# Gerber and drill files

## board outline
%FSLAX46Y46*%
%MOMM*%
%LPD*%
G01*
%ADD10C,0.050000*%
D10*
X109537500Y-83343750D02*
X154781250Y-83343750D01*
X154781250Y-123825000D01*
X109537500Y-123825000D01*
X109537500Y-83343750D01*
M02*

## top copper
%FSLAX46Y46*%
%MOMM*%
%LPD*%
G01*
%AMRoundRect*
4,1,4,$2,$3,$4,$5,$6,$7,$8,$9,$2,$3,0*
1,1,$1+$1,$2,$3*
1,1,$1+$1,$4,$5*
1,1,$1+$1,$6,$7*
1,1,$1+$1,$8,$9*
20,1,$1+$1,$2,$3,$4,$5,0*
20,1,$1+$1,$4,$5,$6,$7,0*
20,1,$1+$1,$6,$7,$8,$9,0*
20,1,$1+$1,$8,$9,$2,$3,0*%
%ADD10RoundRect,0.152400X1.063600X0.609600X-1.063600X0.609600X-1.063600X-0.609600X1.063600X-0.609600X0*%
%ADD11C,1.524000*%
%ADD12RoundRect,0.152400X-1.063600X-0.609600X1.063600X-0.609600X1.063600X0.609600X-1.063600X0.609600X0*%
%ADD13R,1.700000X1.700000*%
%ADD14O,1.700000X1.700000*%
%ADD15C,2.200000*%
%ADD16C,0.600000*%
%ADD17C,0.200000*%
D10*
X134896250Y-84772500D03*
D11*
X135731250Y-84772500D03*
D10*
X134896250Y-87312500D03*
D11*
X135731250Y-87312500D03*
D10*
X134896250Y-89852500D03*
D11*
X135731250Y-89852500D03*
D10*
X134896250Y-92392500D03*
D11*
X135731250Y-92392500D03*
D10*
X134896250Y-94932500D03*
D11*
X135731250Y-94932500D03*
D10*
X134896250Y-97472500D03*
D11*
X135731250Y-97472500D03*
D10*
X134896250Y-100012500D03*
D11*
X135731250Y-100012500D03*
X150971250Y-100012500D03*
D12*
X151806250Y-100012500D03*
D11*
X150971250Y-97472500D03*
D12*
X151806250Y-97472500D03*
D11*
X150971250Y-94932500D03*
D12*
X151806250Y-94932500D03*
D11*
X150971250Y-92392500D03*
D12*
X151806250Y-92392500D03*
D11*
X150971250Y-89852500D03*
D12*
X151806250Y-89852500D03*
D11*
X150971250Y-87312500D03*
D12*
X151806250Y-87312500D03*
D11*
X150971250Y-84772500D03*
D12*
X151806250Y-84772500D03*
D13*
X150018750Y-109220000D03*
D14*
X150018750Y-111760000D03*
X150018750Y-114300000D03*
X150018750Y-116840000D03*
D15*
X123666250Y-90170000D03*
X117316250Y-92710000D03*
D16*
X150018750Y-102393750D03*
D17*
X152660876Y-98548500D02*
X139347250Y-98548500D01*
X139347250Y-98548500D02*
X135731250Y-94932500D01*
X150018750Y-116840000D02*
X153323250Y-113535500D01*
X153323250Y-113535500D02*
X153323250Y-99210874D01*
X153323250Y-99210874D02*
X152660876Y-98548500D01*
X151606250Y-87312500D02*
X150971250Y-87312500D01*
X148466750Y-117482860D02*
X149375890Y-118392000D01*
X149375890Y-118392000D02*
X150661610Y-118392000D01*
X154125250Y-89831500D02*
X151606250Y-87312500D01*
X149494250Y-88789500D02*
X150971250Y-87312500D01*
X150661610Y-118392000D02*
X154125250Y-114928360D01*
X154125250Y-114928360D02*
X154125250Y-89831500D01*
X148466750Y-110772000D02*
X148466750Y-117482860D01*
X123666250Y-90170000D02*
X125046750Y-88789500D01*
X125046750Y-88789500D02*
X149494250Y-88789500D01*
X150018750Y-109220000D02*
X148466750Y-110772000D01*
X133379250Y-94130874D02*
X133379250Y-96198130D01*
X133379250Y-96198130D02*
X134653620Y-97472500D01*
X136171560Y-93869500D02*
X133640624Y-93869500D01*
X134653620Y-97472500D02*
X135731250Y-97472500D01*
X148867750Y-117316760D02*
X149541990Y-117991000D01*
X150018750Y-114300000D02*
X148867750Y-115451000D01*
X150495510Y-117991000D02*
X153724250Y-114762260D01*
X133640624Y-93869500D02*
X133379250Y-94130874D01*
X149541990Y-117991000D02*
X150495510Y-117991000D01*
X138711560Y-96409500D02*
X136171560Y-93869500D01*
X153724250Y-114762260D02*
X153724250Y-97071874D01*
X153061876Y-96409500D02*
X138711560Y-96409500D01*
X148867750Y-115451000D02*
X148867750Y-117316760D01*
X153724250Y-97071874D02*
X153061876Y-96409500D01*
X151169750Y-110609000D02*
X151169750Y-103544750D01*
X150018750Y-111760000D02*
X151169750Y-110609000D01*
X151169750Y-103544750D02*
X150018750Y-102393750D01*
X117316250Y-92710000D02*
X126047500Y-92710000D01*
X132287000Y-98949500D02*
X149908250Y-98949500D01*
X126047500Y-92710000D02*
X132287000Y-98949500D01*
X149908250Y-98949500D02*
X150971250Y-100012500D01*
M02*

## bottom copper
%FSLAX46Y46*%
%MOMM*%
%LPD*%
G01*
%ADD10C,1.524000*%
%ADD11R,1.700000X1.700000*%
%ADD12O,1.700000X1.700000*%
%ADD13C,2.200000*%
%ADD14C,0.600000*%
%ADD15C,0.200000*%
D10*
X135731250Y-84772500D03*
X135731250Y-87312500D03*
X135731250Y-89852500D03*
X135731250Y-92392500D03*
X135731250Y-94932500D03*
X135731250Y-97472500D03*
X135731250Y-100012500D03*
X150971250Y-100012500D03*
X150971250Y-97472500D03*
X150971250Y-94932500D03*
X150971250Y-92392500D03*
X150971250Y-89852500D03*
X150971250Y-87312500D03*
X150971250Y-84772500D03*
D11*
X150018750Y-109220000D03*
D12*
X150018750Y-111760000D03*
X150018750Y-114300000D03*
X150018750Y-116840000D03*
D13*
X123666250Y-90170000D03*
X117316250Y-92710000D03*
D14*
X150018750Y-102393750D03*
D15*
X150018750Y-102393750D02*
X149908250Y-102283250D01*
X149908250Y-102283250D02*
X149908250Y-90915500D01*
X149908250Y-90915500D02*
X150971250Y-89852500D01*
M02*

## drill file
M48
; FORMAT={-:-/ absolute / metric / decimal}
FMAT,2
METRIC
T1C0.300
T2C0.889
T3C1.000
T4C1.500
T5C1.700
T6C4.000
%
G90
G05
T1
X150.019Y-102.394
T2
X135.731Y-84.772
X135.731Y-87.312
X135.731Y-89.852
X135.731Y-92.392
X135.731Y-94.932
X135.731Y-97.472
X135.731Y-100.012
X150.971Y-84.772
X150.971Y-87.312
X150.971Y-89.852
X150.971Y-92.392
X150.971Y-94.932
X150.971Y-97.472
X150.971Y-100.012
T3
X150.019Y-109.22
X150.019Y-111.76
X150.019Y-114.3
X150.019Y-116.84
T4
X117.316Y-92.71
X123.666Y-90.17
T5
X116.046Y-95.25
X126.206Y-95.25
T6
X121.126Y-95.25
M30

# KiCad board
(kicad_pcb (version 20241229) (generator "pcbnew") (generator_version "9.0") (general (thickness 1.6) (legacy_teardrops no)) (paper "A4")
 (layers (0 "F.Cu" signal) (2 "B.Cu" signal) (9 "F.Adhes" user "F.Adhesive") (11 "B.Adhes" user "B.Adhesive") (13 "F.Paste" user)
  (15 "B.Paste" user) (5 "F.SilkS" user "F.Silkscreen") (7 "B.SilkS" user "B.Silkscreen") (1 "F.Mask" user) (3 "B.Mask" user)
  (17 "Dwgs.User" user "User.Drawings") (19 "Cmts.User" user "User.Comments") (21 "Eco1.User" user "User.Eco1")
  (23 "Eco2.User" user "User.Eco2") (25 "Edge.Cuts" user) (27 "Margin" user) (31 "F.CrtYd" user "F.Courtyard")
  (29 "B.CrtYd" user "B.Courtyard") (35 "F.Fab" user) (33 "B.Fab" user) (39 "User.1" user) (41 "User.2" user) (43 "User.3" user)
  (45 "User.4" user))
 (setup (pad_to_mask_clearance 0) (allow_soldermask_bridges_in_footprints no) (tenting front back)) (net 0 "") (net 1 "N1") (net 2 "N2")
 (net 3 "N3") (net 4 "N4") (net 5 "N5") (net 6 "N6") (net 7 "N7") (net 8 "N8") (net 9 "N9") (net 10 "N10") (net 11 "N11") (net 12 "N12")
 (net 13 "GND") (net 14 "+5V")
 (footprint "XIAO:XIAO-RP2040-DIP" (layer "F.Cu") (at 143.35125 92.3925)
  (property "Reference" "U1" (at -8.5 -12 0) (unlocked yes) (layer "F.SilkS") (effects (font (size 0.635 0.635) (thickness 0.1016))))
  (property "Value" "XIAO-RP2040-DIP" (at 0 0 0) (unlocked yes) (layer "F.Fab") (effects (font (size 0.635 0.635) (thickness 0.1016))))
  (pad "1" smd roundrect (at -8.455 -7.62 180) (size 2.432 1.524) (layers "F.Cu" "F.Mask") (roundrect_rratio 0.1) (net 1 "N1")
   (thermal_bridge_angle 45))
  (pad "1" thru_hole circle (at -7.62 -7.62 180) (size 1.524 1.524) (drill 0.889) (layers "*.Cu" "*.Mask") (remove_unused_layers no)
   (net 1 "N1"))
  (pad "2" smd roundrect (at -8.455 -5.08 180) (size 2.432 1.524) (layers "F.Cu" "F.Mask") (roundrect_rratio 0.1) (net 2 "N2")
   (thermal_bridge_angle 45))
  (pad "2" thru_hole circle (at -7.62 -5.08 180) (size 1.524 1.524) (drill 0.889) (layers "*.Cu" "*.Mask") (remove_unused_layers no)
   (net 2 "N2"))
  (pad "3" smd roundrect (at -8.455 -2.54 180) (size 2.432 1.524) (layers "F.Cu" "F.Mask") (roundrect_rratio 0.1) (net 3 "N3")
   (thermal_bridge_angle 45))
  (pad "3" thru_hole circle (at -7.62 -2.54 180) (size 1.524 1.524) (drill 0.889) (layers "*.Cu" "*.Mask") (remove_unused_layers no)
   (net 3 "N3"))
  (pad "4" smd roundrect (at -8.455 0 180) (size 2.432 1.524) (layers "F.Cu" "F.Mask") (roundrect_rratio 0.1) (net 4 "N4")
   (thermal_bridge_angle 45))
  (pad "4" thru_hole circle (at -7.62 0 180) (size 1.524 1.524) (drill 0.889) (layers "*.Cu" "*.Mask") (remove_unused_layers no)
   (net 4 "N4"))
  (pad "5" smd roundrect (at -8.455 2.54 180) (size 2.432 1.524) (layers "F.Cu" "F.Mask") (roundrect_rratio 0.1) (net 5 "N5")
   (thermal_bridge_angle 45))
  (pad "5" thru_hole circle (at -7.62 2.54 180) (size 1.524 1.524) (drill 0.889) (layers "*.Cu" "*.Mask") (remove_unused_layers no)
   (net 5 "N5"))
  (pad "6" smd roundrect (at -8.455 5.08 180) (size 2.432 1.524) (layers "F.Cu" "F.Mask") (roundrect_rratio 0.1) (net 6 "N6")
   (thermal_bridge_angle 45))
  (pad "6" thru_hole circle (at -7.62 5.08 180) (size 1.524 1.524) (drill 0.889) (layers "*.Cu" "*.Mask") (remove_unused_layers no)
   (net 6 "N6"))
  (pad "7" smd roundrect (at -8.455 7.62 180) (size 2.432 1.524) (layers "F.Cu" "F.Mask") (roundrect_rratio 0.1) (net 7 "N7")
   (thermal_bridge_angle 45))
  (pad "7" thru_hole circle (at -7.62 7.62 180) (size 1.524 1.524) (drill 0.889) (layers "*.Cu" "*.Mask") (remove_unused_layers no)
   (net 7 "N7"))
  (pad "8" thru_hole circle (at 7.62 7.62) (size 1.524 1.524) (drill 0.889) (layers "*.Cu" "*.Mask") (remove_unused_layers no) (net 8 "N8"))
  (pad "8" smd roundrect (at 8.455 7.62) (size 2.432 1.524) (layers "F.Cu" "F.Mask") (roundrect_rratio 0.1) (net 8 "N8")
   (thermal_bridge_angle 45))
  (pad "9" thru_hole circle (at 7.62 5.08) (size 1.524 1.524) (drill 0.889) (layers "*.Cu" "*.Mask") (remove_unused_layers no) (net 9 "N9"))
  (pad "9" smd roundrect (at 8.455 5.08) (size 2.432 1.524) (layers "F.Cu" "F.Mask") (roundrect_rratio 0.1) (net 9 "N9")
   (thermal_bridge_angle 45))
  (pad "10" thru_hole circle (at 7.62 2.54) (size 1.524 1.524) (drill 0.889) (layers "*.Cu" "*.Mask") (remove_unused_layers no)
   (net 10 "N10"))
  (pad "10" smd roundrect (at 8.455 2.54) (size 2.432 1.524) (layers "F.Cu" "F.Mask") (roundrect_rratio 0.1) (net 10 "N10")
   (thermal_bridge_angle 45))
  (pad "11" thru_hole circle (at 7.62 0) (size 1.524 1.524) (drill 0.889) (layers "*.Cu" "*.Mask") (remove_unused_layers no) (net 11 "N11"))
  (pad "11" smd roundrect (at 8.455 0) (size 2.432 1.524) (layers "F.Cu" "F.Mask") (roundrect_rratio 0.1) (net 11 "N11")
   (thermal_bridge_angle 45))
  (pad "12" thru_hole circle (at 7.62 -2.54) (size 1.524 1.524) (drill 0.889) (layers "*.Cu" "*.Mask") (remove_unused_layers no)
   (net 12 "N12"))
  (pad "12" smd roundrect (at 8.455 -2.54) (size 2.432 1.524) (layers "F.Cu" "F.Mask") (roundrect_rratio 0.1) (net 12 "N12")
   (thermal_bridge_angle 45))
  (pad "13" thru_hole circle (at 7.62 -5.08) (size 1.524 1.524) (drill 0.889) (layers "*.Cu" "*.Mask") (remove_unused_layers no)
   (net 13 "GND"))
  (pad "13" smd roundrect (at 8.455 -5.08) (size 2.432 1.524) (layers "F.Cu" "F.Mask") (roundrect_rratio 0.1) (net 13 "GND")
   (thermal_bridge_angle 45))
  (pad "14" thru_hole circle (at 7.62 -7.62) (size 1.524 1.524) (drill 0.889) (layers "*.Cu" "*.Mask") (remove_unused_layers no)
   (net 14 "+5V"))
  (pad "14" smd roundrect (at 8.455 -7.62) (size 2.432 1.524) (layers "F.Cu" "F.Mask") (roundrect_rratio 0.1) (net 14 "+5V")
   (thermal_bridge_angle 45)))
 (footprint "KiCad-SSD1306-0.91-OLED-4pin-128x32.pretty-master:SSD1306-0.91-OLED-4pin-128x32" (layer "F.Cu") (at 113.51875 107.03)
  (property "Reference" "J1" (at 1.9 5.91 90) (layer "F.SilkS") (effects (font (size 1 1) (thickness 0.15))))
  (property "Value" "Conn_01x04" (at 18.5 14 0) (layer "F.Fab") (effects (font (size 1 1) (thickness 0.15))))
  (pad "1" thru_hole rect (at 36.5 2.19) (size 1.7 1.7) (drill 1) (layers "*.Cu" "*.Mask") (remove_unused_layers no) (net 13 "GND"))
  (pad "2" thru_hole oval (at 36.5 4.73) (size 1.7 1.7) (drill 1) (layers "*.Cu" "*.Mask") (remove_unused_layers no) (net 12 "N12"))
  (pad "3" thru_hole oval (at 36.5 7.27) (size 1.7 1.7) (drill 1) (layers "*.Cu" "*.Mask") (remove_unused_layers no) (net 6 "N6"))
  (pad "4" thru_hole oval (at 36.5 9.81) (size 1.7 1.7) (drill 1) (layers "*.Cu" "*.Mask") (remove_unused_layers no) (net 5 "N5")))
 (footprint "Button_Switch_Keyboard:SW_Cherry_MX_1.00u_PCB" (layer "F.Cu") (at 123.66625 90.17)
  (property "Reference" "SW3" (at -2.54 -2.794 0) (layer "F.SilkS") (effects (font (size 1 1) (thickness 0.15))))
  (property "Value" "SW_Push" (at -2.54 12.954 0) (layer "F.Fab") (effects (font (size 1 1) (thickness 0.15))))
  (pad "" np_thru_hole circle (at -7.62 5.08) (size 1.7 1.7) (drill 1.7) (layers "*.Cu" "*.Mask"))
  (pad "" np_thru_hole circle (at -2.54 5.08) (size 4 4) (drill 4) (layers "*.Cu" "*.Mask"))
  (pad "" np_thru_hole circle (at 2.54 5.08) (size 1.7 1.7) (drill 1.7) (layers "*.Cu" "*.Mask"))
  (pad "1" thru_hole circle (at 0 0) (size 2.2 2.2) (drill 1.5) (layers "*.Cu" "*.Mask") (remove_unused_layers no) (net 13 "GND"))
  (pad "2" thru_hole circle (at -6.35 2.54) (size 2.2 2.2) (drill 1.5) (layers "*.Cu" "*.Mask") (remove_unused_layers no) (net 8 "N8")))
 (gr_rect (start 109.5375 83.34375) (end 154.78125 123.825) (stroke (width 0.05) (type default)) (fill no) (layer "Edge.Cuts"))
 (segment (start 152.660876 98.5485) (end 139.34725 98.5485) (width 0.2) (layer "F.Cu") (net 5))
 (segment (start 139.34725 98.5485) (end 135.73125 94.9325) (width 0.2) (layer "F.Cu") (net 5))
 (segment (start 150.01875 116.84) (end 153.32325 113.5355) (width 0.2) (layer "F.Cu") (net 5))
 (segment (start 153.32325 113.5355) (end 153.32325 99.210874) (width 0.2) (layer "F.Cu") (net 5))
 (segment (start 153.32325 99.210874) (end 152.660876 98.5485) (width 0.2) (layer "F.Cu") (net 5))
 (segment (start 151.60625 87.3125) (end 150.97125 87.3125) (width 0.2) (layer "F.Cu") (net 13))
 (segment (start 148.46675 117.48286) (end 149.37589 118.392) (width 0.2) (layer "F.Cu") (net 13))
 (segment (start 149.37589 118.392) (end 150.66161 118.392) (width 0.2) (layer "F.Cu") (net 13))
 (segment (start 154.12525 89.8315) (end 151.60625 87.3125) (width 0.2) (layer "F.Cu") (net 13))
 (segment (start 149.49425 88.7895) (end 150.97125 87.3125) (width 0.2) (layer "F.Cu") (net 13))
 (segment (start 150.66161 118.392) (end 154.12525 114.92836) (width 0.2) (layer "F.Cu") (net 13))
 (segment (start 154.12525 114.92836) (end 154.12525 89.8315) (width 0.2) (layer "F.Cu") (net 13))
 (segment (start 148.46675 110.772) (end 148.46675 117.48286) (width 0.2) (layer "F.Cu") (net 13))
 (segment (start 123.66625 90.17) (end 125.04675 88.7895) (width 0.2) (layer "F.Cu") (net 13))
 (segment (start 125.04675 88.7895) (end 149.49425 88.7895) (width 0.2) (layer "F.Cu") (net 13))
 (segment (start 150.01875 109.22) (end 148.46675 110.772) (width 0.2) (layer "F.Cu") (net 13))
 (segment (start 133.37925 94.130874) (end 133.37925 96.19813) (width 0.2) (layer "F.Cu") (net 6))
 (segment (start 133.37925 96.19813) (end 134.65362 97.4725) (width 0.2) (layer "F.Cu") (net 6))
 (segment (start 136.17156 93.8695) (end 133.640624 93.8695) (width 0.2) (layer "F.Cu") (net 6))
 (segment (start 134.65362 97.4725) (end 135.73125 97.4725) (width 0.2) (layer "F.Cu") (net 6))
 (segment (start 148.86775 117.31676) (end 149.54199 117.991) (width 0.2) (layer "F.Cu") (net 6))
 (segment (start 150.01875 114.3) (end 148.86775 115.451) (width 0.2) (layer "F.Cu") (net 6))
 (segment (start 150.49551 117.991) (end 153.72425 114.76226) (width 0.2) (layer "F.Cu") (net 6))
 (segment (start 133.640624 93.8695) (end 133.37925 94.130874) (width 0.2) (layer "F.Cu") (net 6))
 (segment (start 149.54199 117.991) (end 150.49551 117.991) (width 0.2) (layer "F.Cu") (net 6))
 (segment (start 138.71156 96.4095) (end 136.17156 93.8695) (width 0.2) (layer "F.Cu") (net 6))
 (segment (start 153.72425 114.76226) (end 153.72425 97.071874) (width 0.2) (layer "F.Cu") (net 6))
 (segment (start 153.061876 96.4095) (end 138.71156 96.4095) (width 0.2) (layer "F.Cu") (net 6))
 (segment (start 148.86775 115.451) (end 148.86775 117.31676) (width 0.2) (layer "F.Cu") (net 6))
 (segment (start 153.72425 97.071874) (end 153.061876 96.4095) (width 0.2) (layer "F.Cu") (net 6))
 (segment (start 151.16975 110.609) (end 151.16975 103.54475) (width 0.2) (layer "F.Cu") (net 12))
 (segment (start 150.01875 111.76) (end 151.16975 110.609) (width 0.2) (layer "F.Cu") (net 12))
 (segment (start 151.16975 103.54475) (end 150.01875 102.39375) (width 0.2) (layer "F.Cu") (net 12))
 (via (at 150.01875 102.39375) (size 0.6) (drill 0.3) (layers "F.Cu" "B.Cu") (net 12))
 (segment (start 150.01875 102.39375) (end 149.90825 102.28325) (width 0.2) (layer "B.Cu") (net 12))
 (segment (start 149.90825 102.28325) (end 149.90825 90.9155) (width 0.2) (layer "B.Cu") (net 12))
 (segment (start 149.90825 90.9155) (end 150.97125 89.8525) (width 0.2) (layer "B.Cu") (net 12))
 (segment (start 117.31625 92.71) (end 126.0475 92.71) (width 0.2) (layer "F.Cu") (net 8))
 (segment (start 132.287 98.9495) (end 149.90825 98.9495) (width 0.2) (layer "F.Cu") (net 8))
 (segment (start 126.0475 92.71) (end 132.287 98.9495) (width 0.2) (layer "F.Cu") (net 8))
 (segment (start 149.90825 98.9495) (end 150.97125 100.0125) (width 0.2) (layer "F.Cu") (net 8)))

